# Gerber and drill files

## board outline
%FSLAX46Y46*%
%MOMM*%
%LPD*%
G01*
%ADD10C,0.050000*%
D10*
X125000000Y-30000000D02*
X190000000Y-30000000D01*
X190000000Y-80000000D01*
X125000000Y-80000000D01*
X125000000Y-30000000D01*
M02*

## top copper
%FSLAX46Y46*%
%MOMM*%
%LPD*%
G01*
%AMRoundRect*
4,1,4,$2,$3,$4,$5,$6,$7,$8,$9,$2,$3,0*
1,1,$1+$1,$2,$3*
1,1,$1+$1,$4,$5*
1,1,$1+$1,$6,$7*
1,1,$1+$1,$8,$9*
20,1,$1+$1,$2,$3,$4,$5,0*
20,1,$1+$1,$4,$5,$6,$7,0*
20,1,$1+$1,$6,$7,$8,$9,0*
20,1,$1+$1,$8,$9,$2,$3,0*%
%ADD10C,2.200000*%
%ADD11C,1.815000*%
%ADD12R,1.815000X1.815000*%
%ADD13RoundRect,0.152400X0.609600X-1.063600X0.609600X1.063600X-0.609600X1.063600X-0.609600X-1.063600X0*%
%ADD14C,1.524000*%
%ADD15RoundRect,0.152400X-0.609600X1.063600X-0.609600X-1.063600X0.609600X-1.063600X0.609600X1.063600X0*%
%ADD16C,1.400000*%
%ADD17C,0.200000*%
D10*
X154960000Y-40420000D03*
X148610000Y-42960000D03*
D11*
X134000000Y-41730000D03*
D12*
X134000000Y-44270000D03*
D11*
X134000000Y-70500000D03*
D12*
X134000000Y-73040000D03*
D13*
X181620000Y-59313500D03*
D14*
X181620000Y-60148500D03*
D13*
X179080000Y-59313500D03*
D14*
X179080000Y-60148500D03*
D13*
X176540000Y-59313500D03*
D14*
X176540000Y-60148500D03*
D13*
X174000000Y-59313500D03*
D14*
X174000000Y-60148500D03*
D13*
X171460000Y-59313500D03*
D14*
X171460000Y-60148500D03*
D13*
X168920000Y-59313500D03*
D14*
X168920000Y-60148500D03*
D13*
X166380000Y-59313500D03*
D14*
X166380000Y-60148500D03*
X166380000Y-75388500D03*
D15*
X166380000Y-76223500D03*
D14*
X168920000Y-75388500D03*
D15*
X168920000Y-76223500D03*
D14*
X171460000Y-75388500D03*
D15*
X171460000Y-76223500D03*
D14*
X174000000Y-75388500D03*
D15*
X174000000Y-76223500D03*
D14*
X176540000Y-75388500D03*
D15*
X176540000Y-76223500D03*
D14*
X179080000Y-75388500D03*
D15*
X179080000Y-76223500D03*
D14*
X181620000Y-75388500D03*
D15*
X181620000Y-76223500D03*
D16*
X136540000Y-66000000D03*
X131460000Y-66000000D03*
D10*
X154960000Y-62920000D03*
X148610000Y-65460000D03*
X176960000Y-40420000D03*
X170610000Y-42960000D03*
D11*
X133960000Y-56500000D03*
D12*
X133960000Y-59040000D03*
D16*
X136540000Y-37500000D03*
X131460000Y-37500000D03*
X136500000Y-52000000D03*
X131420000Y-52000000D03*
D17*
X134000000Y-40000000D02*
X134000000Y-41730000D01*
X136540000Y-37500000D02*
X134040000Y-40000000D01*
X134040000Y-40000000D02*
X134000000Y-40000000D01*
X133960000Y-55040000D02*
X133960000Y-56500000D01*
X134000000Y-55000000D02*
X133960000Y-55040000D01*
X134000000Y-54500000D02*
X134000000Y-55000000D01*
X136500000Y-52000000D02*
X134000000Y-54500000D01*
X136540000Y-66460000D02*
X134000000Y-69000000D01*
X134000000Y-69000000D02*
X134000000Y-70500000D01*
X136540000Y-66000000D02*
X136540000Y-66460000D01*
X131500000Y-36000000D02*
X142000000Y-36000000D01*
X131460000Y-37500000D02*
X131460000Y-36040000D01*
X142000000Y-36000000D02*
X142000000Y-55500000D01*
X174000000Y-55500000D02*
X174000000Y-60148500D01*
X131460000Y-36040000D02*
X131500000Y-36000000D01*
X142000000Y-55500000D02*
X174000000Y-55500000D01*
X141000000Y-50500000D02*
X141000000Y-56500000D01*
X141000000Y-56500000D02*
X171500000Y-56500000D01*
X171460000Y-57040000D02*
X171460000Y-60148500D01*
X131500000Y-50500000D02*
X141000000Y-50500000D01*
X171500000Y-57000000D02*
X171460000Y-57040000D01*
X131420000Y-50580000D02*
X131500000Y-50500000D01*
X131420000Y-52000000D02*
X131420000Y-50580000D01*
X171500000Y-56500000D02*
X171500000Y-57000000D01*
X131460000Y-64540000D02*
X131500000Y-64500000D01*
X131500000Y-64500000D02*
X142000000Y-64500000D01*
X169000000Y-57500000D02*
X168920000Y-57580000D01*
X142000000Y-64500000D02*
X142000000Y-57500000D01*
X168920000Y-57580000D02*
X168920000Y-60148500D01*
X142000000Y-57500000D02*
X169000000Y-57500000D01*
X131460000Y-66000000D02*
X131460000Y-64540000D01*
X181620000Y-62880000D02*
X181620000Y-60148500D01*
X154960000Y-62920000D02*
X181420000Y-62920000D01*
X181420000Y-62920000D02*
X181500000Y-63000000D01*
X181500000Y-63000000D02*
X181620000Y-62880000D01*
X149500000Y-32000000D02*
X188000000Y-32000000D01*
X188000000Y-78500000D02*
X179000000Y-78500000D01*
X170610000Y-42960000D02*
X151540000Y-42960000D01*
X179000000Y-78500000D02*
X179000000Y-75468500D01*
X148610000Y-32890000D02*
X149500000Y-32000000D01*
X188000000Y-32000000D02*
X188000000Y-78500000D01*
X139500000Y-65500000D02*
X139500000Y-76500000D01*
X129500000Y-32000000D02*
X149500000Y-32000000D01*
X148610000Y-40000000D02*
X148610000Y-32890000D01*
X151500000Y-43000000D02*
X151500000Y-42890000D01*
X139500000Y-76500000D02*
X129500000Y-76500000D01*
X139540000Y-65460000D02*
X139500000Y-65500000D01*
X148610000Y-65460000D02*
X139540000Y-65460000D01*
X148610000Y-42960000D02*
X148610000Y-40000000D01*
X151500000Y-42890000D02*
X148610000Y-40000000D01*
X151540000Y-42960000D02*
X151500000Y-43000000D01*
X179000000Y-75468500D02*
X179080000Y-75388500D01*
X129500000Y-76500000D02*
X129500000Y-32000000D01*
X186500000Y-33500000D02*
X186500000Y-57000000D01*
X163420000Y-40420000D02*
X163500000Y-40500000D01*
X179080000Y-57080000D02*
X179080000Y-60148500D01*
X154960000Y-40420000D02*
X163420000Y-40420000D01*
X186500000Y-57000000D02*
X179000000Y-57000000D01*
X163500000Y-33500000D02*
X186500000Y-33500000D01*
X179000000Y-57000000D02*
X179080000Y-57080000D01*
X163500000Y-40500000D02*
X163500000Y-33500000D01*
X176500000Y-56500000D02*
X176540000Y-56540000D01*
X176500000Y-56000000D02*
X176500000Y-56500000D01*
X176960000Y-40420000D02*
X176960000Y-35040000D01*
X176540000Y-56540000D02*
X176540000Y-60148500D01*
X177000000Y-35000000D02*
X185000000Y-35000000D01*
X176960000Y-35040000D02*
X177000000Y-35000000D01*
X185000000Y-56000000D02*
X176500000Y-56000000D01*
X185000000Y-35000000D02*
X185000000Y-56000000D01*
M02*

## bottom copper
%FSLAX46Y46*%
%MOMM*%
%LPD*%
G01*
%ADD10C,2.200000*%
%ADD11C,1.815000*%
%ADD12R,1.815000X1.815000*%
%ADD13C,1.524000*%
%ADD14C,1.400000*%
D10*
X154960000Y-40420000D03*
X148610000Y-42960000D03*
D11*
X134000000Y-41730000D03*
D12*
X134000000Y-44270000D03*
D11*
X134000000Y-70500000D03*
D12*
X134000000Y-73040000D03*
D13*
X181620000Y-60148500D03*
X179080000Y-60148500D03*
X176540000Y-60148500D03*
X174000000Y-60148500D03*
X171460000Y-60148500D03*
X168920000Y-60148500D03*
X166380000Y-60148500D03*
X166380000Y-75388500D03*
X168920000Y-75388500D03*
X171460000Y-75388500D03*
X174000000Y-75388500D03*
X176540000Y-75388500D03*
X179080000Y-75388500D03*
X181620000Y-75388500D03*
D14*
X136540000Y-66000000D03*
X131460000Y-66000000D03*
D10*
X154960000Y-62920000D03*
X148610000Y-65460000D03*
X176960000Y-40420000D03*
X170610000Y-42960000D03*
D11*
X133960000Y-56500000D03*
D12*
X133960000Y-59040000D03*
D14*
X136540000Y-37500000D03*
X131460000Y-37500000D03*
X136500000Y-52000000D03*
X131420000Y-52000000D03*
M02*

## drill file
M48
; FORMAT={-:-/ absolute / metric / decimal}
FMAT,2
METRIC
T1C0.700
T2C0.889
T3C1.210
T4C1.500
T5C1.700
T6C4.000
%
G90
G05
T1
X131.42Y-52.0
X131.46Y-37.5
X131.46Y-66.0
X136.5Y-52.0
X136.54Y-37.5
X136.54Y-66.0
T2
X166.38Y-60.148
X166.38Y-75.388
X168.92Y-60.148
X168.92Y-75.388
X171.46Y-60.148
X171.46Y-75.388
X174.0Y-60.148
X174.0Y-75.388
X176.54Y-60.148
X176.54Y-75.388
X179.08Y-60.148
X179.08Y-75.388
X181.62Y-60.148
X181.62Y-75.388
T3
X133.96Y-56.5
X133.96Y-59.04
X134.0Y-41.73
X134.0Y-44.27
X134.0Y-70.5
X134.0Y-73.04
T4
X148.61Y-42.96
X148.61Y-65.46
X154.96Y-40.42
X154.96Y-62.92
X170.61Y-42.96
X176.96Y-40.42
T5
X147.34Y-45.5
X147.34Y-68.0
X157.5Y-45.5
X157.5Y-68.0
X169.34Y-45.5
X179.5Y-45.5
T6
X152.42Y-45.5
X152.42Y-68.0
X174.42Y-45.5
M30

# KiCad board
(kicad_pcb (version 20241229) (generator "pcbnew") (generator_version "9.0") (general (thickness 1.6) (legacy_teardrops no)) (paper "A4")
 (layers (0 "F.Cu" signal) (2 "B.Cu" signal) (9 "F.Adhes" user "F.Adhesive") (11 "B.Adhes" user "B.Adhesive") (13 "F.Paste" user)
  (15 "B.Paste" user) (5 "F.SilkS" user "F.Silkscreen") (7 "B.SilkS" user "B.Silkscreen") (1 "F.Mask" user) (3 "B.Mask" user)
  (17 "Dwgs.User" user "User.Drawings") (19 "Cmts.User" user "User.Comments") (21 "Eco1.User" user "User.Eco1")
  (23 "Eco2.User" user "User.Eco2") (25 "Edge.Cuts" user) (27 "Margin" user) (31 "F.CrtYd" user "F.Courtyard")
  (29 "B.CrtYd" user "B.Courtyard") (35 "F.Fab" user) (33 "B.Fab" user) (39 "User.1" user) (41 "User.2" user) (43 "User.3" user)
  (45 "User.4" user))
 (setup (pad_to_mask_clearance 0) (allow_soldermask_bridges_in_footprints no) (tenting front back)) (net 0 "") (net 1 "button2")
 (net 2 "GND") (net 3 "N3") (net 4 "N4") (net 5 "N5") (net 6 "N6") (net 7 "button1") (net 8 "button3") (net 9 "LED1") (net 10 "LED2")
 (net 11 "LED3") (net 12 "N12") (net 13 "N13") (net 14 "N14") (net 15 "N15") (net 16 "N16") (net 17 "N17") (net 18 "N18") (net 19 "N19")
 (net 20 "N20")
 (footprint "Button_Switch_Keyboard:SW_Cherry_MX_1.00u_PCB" (layer "F.Cu") (at 154.96 40.42)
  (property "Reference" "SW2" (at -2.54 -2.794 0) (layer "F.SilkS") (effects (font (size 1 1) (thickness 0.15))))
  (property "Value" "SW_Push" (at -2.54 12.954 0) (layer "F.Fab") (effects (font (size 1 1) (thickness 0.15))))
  (pad "" np_thru_hole circle (at -7.62 5.08) (size 1.7 1.7) (drill 1.7) (layers "*.Cu" "*.Mask"))
  (pad "" np_thru_hole circle (at -2.54 5.08) (size 4 4) (drill 4) (layers "*.Cu" "*.Mask"))
  (pad "" np_thru_hole circle (at 2.54 5.08) (size 1.7 1.7) (drill 1.7) (layers "*.Cu" "*.Mask"))
  (pad "1" thru_hole circle (at 0 0) (size 2.2 2.2) (drill 1.5) (layers "*.Cu" "*.Mask") (remove_unused_layers no) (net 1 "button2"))
  (pad "2" thru_hole circle (at -6.35 2.54) (size 2.2 2.2) (drill 1.5) (layers "*.Cu" "*.Mask") (remove_unused_layers no) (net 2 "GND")))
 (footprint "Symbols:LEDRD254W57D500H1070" (layer "F.Cu") (at 134 43 90)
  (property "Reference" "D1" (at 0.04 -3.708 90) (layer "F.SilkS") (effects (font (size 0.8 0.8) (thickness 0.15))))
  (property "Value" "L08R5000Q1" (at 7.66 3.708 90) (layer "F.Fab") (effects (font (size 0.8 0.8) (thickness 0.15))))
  (pad "A" thru_hole circle (at 1.27 0 90) (size 1.815 1.815) (drill 1.21) (layers "*.Cu" "*.Mask") (remove_unused_layers no) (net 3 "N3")
   (solder_mask_margin 0.102))
  (pad "C" thru_hole rect (at -1.27 0 90) (size 1.815 1.815) (drill 1.21) (layers "*.Cu" "*.Mask") (remove_unused_layers no) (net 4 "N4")
   (solder_mask_margin 0.102)))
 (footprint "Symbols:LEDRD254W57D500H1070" (layer "F.Cu") (at 134 71.77 90)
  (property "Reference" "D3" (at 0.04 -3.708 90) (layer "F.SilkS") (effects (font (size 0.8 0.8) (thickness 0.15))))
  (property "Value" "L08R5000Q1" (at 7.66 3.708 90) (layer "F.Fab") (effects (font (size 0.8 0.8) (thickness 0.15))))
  (pad "A" thru_hole circle (at 1.27 0 90) (size 1.815 1.815) (drill 1.21) (layers "*.Cu" "*.Mask") (remove_unused_layers no) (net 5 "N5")
   (solder_mask_margin 0.102))
  (pad "C" thru_hole rect (at -1.27 0 90) (size 1.815 1.815) (drill 1.21) (layers "*.Cu" "*.Mask") (remove_unused_layers no) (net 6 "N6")
   (solder_mask_margin 0.102)))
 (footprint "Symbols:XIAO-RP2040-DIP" (layer "F.Cu") (at 174 67.7685 -90)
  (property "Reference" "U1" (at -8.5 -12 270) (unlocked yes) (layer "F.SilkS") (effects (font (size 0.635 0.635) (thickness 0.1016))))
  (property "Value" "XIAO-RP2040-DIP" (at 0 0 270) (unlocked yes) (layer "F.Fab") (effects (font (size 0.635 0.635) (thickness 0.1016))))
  (pad "1" smd roundrect (at -8.455 -7.62 90) (size 2.432 1.524) (layers "F.Cu" "F.Mask") (roundrect_rratio 0.1) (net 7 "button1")
   (thermal_bridge_angle 45))
  (pad "1" thru_hole circle (at -7.62 -7.62 90) (size 1.524 1.524) (drill 0.889) (layers "*.Cu" "*.Mask") (remove_unused_layers no)
   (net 7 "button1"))
  (pad "2" smd roundrect (at -8.455 -5.08 90) (size 2.432 1.524) (layers "F.Cu" "F.Mask") (roundrect_rratio 0.1) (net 1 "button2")
   (thermal_bridge_angle 45))
  (pad "2" thru_hole circle (at -7.62 -5.08 90) (size 1.524 1.524) (drill 0.889) (layers "*.Cu" "*.Mask") (remove_unused_layers no)
   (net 1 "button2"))
  (pad "3" smd roundrect (at -8.455 -2.54 90) (size 2.432 1.524) (layers "F.Cu" "F.Mask") (roundrect_rratio 0.1) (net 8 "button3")
   (thermal_bridge_angle 45))
  (pad "3" thru_hole circle (at -7.62 -2.54 90) (size 1.524 1.524) (drill 0.889) (layers "*.Cu" "*.Mask") (remove_unused_layers no)
   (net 8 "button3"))
  (pad "4" smd roundrect (at -8.455 0 90) (size 2.432 1.524) (layers "F.Cu" "F.Mask") (roundrect_rratio 0.1) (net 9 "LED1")
   (thermal_bridge_angle 45))
  (pad "4" thru_hole circle (at -7.62 0 90) (size 1.524 1.524) (drill 0.889) (layers "*.Cu" "*.Mask") (remove_unused_layers no)
   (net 9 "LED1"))
  (pad "5" smd roundrect (at -8.455 2.54 90) (size 2.432 1.524) (layers "F.Cu" "F.Mask") (roundrect_rratio 0.1) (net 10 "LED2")
   (thermal_bridge_angle 45))
  (pad "5" thru_hole circle (at -7.62 2.54 90) (size 1.524 1.524) (drill 0.889) (layers "*.Cu" "*.Mask") (remove_unused_layers no)
   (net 10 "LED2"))
  (pad "6" smd roundrect (at -8.455 5.08 90) (size 2.432 1.524) (layers "F.Cu" "F.Mask") (roundrect_rratio 0.1) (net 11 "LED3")
   (thermal_bridge_angle 45))
  (pad "6" thru_hole circle (at -7.62 5.08 90) (size 1.524 1.524) (drill 0.889) (layers "*.Cu" "*.Mask") (remove_unused_layers no)
   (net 11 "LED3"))
  (pad "7" smd roundrect (at -8.455 7.62 90) (size 2.432 1.524) (layers "F.Cu" "F.Mask") (roundrect_rratio 0.1) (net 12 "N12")
   (thermal_bridge_angle 45))
  (pad "7" thru_hole circle (at -7.62 7.62 90) (size 1.524 1.524) (drill 0.889) (layers "*.Cu" "*.Mask") (remove_unused_layers no)
   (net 12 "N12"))
  (pad "8" thru_hole circle (at 7.62 7.62 270) (size 1.524 1.524) (drill 0.889) (layers "*.Cu" "*.Mask") (remove_unused_layers no)
   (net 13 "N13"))
  (pad "8" smd roundrect (at 8.455 7.62 270) (size 2.432 1.524) (layers "F.Cu" "F.Mask") (roundrect_rratio 0.1) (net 13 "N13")
   (thermal_bridge_angle 45))
  (pad "9" thru_hole circle (at 7.62 5.08 270) (size 1.524 1.524) (drill 0.889) (layers "*.Cu" "*.Mask") (remove_unused_layers no)
   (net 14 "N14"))
  (pad "9" smd roundrect (at 8.455 5.08 270) (size 2.432 1.524) (layers "F.Cu" "F.Mask") (roundrect_rratio 0.1) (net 14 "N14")
   (thermal_bridge_angle 45))
  (pad "10" thru_hole circle (at 7.62 2.54 270) (size 1.524 1.524) (drill 0.889) (layers "*.Cu" "*.Mask") (remove_unused_layers no)
   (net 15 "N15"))
  (pad "10" smd roundrect (at 8.455 2.54 270) (size 2.432 1.524) (layers "F.Cu" "F.Mask") (roundrect_rratio 0.1) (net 15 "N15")
   (thermal_bridge_angle 45))
  (pad "11" thru_hole circle (at 7.62 0 270) (size 1.524 1.524) (drill 0.889) (layers "*.Cu" "*.Mask") (remove_unused_layers no)
   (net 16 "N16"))
  (pad "11" smd roundrect (at 8.455 0 270) (size 2.432 1.524) (layers "F.Cu" "F.Mask") (roundrect_rratio 0.1) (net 16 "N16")
   (thermal_bridge_angle 45))
  (pad "12" thru_hole circle (at 7.62 -2.54 270) (size 1.524 1.524) (drill 0.889) (layers "*.Cu" "*.Mask") (remove_unused_layers no)
   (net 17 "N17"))
  (pad "12" smd roundrect (at 8.455 -2.54 270) (size 2.432 1.524) (layers "F.Cu" "F.Mask") (roundrect_rratio 0.1) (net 17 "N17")
   (thermal_bridge_angle 45))
  (pad "13" thru_hole circle (at 7.62 -5.08 270) (size 1.524 1.524) (drill 0.889) (layers "*.Cu" "*.Mask") (remove_unused_layers no)
   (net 2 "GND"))
  (pad "13" smd roundrect (at 8.455 -5.08 270) (size 2.432 1.524) (layers "F.Cu" "F.Mask") (roundrect_rratio 0.1) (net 2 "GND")
   (thermal_bridge_angle 45))
  (pad "14" thru_hole circle (at 7.62 -7.62 270) (size 1.524 1.524) (drill 0.889) (layers "*.Cu" "*.Mask") (remove_unused_layers no)
   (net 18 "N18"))
  (pad "14" smd roundrect (at 8.455 -7.62 270) (size 2.432 1.524) (layers "F.Cu" "F.Mask") (roundrect_rratio 0.1) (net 18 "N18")
   (thermal_bridge_angle 45)))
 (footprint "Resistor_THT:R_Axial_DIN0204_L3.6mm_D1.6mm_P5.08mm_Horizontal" (layer "F.Cu") (at 136.54 66 180)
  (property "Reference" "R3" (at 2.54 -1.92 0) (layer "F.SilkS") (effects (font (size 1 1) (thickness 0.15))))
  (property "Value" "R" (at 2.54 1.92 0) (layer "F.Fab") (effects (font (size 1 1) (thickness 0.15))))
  (pad "1" thru_hole circle (at 0 0 180) (size 1.4 1.4) (drill 0.7) (layers "*.Cu" "*.Mask") (remove_unused_layers no) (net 5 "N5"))
  (pad "2" thru_hole circle (at 5.08 0 180) (size 1.4 1.4) (drill 0.7) (layers "*.Cu" "*.Mask") (remove_unused_layers no) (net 11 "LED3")))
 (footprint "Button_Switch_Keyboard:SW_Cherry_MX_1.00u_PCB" (layer "F.Cu") (at 154.96 62.92)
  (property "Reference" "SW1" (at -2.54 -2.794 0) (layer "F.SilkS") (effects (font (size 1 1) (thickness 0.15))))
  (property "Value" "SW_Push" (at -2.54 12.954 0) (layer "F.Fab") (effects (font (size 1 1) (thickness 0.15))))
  (pad "" np_thru_hole circle (at -7.62 5.08) (size 1.7 1.7) (drill 1.7) (layers "*.Cu" "*.Mask"))
  (pad "" np_thru_hole circle (at -2.54 5.08) (size 4 4) (drill 4) (layers "*.Cu" "*.Mask"))
  (pad "" np_thru_hole circle (at 2.54 5.08) (size 1.7 1.7) (drill 1.7) (layers "*.Cu" "*.Mask"))
  (pad "1" thru_hole circle (at 0 0) (size 2.2 2.2) (drill 1.5) (layers "*.Cu" "*.Mask") (remove_unused_layers no) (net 7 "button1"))
  (pad "2" thru_hole circle (at -6.35 2.54) (size 2.2 2.2) (drill 1.5) (layers "*.Cu" "*.Mask") (remove_unused_layers no) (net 2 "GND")))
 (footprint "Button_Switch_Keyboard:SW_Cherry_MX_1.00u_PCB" (layer "F.Cu") (at 176.96 40.42)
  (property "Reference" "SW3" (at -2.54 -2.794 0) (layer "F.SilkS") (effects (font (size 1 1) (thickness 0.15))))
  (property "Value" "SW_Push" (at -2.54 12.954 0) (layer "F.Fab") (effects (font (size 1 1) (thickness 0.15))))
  (pad "" np_thru_hole circle (at -7.62 5.08) (size 1.7 1.7) (drill 1.7) (layers "*.Cu" "*.Mask"))
  (pad "" np_thru_hole circle (at -2.54 5.08) (size 4 4) (drill 4) (layers "*.Cu" "*.Mask"))
  (pad "" np_thru_hole circle (at 2.54 5.08) (size 1.7 1.7) (drill 1.7) (layers "*.Cu" "*.Mask"))
  (pad "1" thru_hole circle (at 0 0) (size 2.2 2.2) (drill 1.5) (layers "*.Cu" "*.Mask") (remove_unused_layers no) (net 8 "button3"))
  (pad "2" thru_hole circle (at -6.35 2.54) (size 2.2 2.2) (drill 1.5) (layers "*.Cu" "*.Mask") (remove_unused_layers no) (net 2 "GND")))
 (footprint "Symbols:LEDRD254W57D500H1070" (layer "F.Cu") (at 133.96 57.77 90)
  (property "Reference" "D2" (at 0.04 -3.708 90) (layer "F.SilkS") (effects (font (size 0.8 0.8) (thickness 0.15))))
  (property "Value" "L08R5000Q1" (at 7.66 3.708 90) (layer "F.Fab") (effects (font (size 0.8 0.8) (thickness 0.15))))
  (pad "A" thru_hole circle (at 1.27 0 90) (size 1.815 1.815) (drill 1.21) (layers "*.Cu" "*.Mask") (remove_unused_layers no) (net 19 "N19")
   (solder_mask_margin 0.102))
  (pad "C" thru_hole rect (at -1.27 0 90) (size 1.815 1.815) (drill 1.21) (layers "*.Cu" "*.Mask") (remove_unused_layers no) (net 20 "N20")
   (solder_mask_margin 0.102)))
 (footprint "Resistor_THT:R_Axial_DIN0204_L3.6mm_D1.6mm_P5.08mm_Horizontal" (layer "F.Cu") (at 136.54 37.5 180)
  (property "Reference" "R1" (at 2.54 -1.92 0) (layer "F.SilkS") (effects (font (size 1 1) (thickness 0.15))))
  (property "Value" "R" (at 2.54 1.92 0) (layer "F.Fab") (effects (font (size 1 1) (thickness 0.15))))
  (pad "1" thru_hole circle (at 0 0 180) (size 1.4 1.4) (drill 0.7) (layers "*.Cu" "*.Mask") (remove_unused_layers no) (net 3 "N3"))
  (pad "2" thru_hole circle (at 5.08 0 180) (size 1.4 1.4) (drill 0.7) (layers "*.Cu" "*.Mask") (remove_unused_layers no) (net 9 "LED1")))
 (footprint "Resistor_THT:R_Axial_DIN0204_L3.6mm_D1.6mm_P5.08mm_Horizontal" (layer "F.Cu") (at 136.5 52 180)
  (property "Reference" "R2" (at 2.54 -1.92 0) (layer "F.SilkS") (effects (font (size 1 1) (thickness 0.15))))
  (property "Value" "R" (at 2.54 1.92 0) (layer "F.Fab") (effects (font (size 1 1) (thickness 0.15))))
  (pad "1" thru_hole circle (at 0 0 180) (size 1.4 1.4) (drill 0.7) (layers "*.Cu" "*.Mask") (remove_unused_layers no) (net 19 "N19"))
  (pad "2" thru_hole circle (at 5.08 0 180) (size 1.4 1.4) (drill 0.7) (layers "*.Cu" "*.Mask") (remove_unused_layers no) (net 10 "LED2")))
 (gr_rect (start 125 30) (end 190 80) (stroke (width 0.05) (type default)) (fill no) (layer "Edge.Cuts"))
 (segment (start 134 40) (end 134 41.73) (width 0.2) (layer "F.Cu") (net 3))
 (segment (start 136.54 37.5) (end 134.04 40) (width 0.2) (layer "F.Cu") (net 3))
 (segment (start 134.04 40) (end 134 40) (width 0.2) (layer "F.Cu") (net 3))
 (segment (start 133.96 55.04) (end 133.96 56.5) (width 0.2) (layer "F.Cu") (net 19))
 (segment (start 134 55) (end 133.96 55.04) (width 0.2) (layer "F.Cu") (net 19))
 (segment (start 134 54.5) (end 134 55) (width 0.2) (layer "F.Cu") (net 19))
 (segment (start 136.5 52) (end 134 54.5) (width 0.2) (layer "F.Cu") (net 19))
 (segment (start 136.54 66.46) (end 134 69) (width 0.2) (layer "F.Cu") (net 5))
 (segment (start 134 69) (end 134 70.5) (width 0.2) (layer "F.Cu") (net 5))
 (segment (start 136.54 66) (end 136.54 66.46) (width 0.2) (layer "F.Cu") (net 5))
 (segment (start 131.5 36) (end 142 36) (width 0.2) (layer "F.Cu") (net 9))
 (segment (start 131.46 37.5) (end 131.46 36.04) (width 0.2) (layer "F.Cu") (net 9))
 (segment (start 142 36) (end 142 55.5) (width 0.2) (layer "F.Cu") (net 9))
 (segment (start 174 55.5) (end 174 60.1485) (width 0.2) (layer "F.Cu") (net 9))
 (segment (start 131.46 36.04) (end 131.5 36) (width 0.2) (layer "F.Cu") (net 9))
 (segment (start 142 55.5) (end 174 55.5) (width 0.2) (layer "F.Cu") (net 9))
 (segment (start 141 50.5) (end 141 56.5) (width 0.2) (layer "F.Cu") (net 10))
 (segment (start 141 56.5) (end 171.5 56.5) (width 0.2) (layer "F.Cu") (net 10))
 (segment (start 171.46 57.04) (end 171.46 60.1485) (width 0.2) (layer "F.Cu") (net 10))
 (segment (start 131.5 50.5) (end 141 50.5) (width 0.2) (layer "F.Cu") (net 10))
 (segment (start 171.5 57) (end 171.46 57.04) (width 0.2) (layer "F.Cu") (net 10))
 (segment (start 131.42 50.58) (end 131.5 50.5) (width 0.2) (layer "F.Cu") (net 10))
 (segment (start 131.42 52) (end 131.42 50.58) (width 0.2) (layer "F.Cu") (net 10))
 (segment (start 171.5 56.5) (end 171.5 57) (width 0.2) (layer "F.Cu") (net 10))
 (segment (start 131.46 64.54) (end 131.5 64.5) (width 0.2) (layer "F.Cu") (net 11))
 (segment (start 131.5 64.5) (end 142 64.5) (width 0.2) (layer "F.Cu") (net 11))
 (segment (start 169 57.5) (end 168.92 57.58) (width 0.2) (layer "F.Cu") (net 11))
 (segment (start 142 64.5) (end 142 57.5) (width 0.2) (layer "F.Cu") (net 11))
 (segment (start 168.92 57.58) (end 168.92 60.1485) (width 0.2) (layer "F.Cu") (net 11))
 (segment (start 142 57.5) (end 169 57.5) (width 0.2) (layer "F.Cu") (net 11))
 (segment (start 131.46 66) (end 131.46 64.54) (width 0.2) (layer "F.Cu") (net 11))
 (segment (start 181.62 62.88) (end 181.62 60.1485) (width 0.2) (layer "F.Cu") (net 7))
 (segment (start 154.96 62.92) (end 181.42 62.92) (width 0.2) (layer "F.Cu") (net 7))
 (segment (start 181.42 62.92) (end 181.5 63) (width 0.2) (layer "F.Cu") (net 7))
 (segment (start 181.5 63) (end 181.62 62.88) (width 0.2) (layer "F.Cu") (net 7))
 (segment (start 149.5 32) (end 188 32) (width 0.2) (layer "F.Cu") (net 2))
 (segment (start 188 78.5) (end 179 78.5) (width 0.2) (layer "F.Cu") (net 2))
 (segment (start 170.61 42.96) (end 151.54 42.96) (width 0.2) (layer "F.Cu") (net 2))
 (segment (start 179 78.5) (end 179 75.4685) (width 0.2) (layer "F.Cu") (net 2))
 (segment (start 148.61 32.89) (end 149.5 32) (width 0.2) (layer "F.Cu") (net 2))
 (segment (start 188 32) (end 188 78.5) (width 0.2) (layer "F.Cu") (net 2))
 (segment (start 139.5 65.5) (end 139.5 76.5) (width 0.2) (layer "F.Cu") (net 2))
 (segment (start 129.5 32) (end 149.5 32) (width 0.2) (layer "F.Cu") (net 2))
 (segment (start 148.61 40) (end 148.61 32.89) (width 0.2) (layer "F.Cu") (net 2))
 (segment (start 151.5 43) (end 151.5 42.89) (width 0.2) (layer "F.Cu") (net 2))
 (segment (start 139.5 76.5) (end 129.5 76.5) (width 0.2) (layer "F.Cu") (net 2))
 (segment (start 139.54 65.46) (end 139.5 65.5) (width 0.2) (layer "F.Cu") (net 2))
 (segment (start 148.61 65.46) (end 139.54 65.46) (width 0.2) (layer "F.Cu") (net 2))
 (segment (start 148.61 42.96) (end 148.61 40) (width 0.2) (layer "F.Cu") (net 2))
 (segment (start 151.5 42.89) (end 148.61 40) (width 0.2) (layer "F.Cu") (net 2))
 (segment (start 151.54 42.96) (end 151.5 43) (width 0.2) (layer "F.Cu") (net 2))
 (segment (start 179 75.4685) (end 179.08 75.3885) (width 0.2) (layer "F.Cu") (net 2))
 (segment (start 129.5 76.5) (end 129.5 32) (width 0.2) (layer "F.Cu") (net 2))
 (segment (start 186.5 33.5) (end 186.5 57) (width 0.2) (layer "F.Cu") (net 1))
 (segment (start 163.42 40.42) (end 163.5 40.5) (width 0.2) (layer "F.Cu") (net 1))
 (segment (start 179.08 57.08) (end 179.08 60.1485) (width 0.2) (layer "F.Cu") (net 1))
 (segment (start 154.96 40.42) (end 163.42 40.42) (width 0.2) (layer "F.Cu") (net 1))
 (segment (start 186.5 57) (end 179 57) (width 0.2) (layer "F.Cu") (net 1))
 (segment (start 163.5 33.5) (end 186.5 33.5) (width 0.2) (layer "F.Cu") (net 1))
 (segment (start 179 57) (end 179.08 57.08) (width 0.2) (layer "F.Cu") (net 1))
 (segment (start 163.5 40.5) (end 163.5 33.5) (width 0.2) (layer "F.Cu") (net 1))
 (segment (start 176.5 56.5) (end 176.54 56.54) (width 0.2) (layer "F.Cu") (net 8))
 (segment (start 176.5 56) (end 176.5 56.5) (width 0.2) (layer "F.Cu") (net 8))
 (segment (start 176.96 40.42) (end 176.96 35.04) (width 0.2) (layer "F.Cu") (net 8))
 (segment (start 176.54 56.54) (end 176.54 60.1485) (width 0.2) (layer "F.Cu") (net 8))
 (segment (start 177 35) (end 185 35) (width 0.2) (layer "F.Cu") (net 8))
 (segment (start 176.96 35.04) (end 177 35) (width 0.2) (layer "F.Cu") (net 8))
 (segment (start 185 56) (end 176.5 56) (width 0.2) (layer "F.Cu") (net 8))
 (segment (start 185 35) (end 185 56) (width 0.2) (layer "F.Cu") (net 8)))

